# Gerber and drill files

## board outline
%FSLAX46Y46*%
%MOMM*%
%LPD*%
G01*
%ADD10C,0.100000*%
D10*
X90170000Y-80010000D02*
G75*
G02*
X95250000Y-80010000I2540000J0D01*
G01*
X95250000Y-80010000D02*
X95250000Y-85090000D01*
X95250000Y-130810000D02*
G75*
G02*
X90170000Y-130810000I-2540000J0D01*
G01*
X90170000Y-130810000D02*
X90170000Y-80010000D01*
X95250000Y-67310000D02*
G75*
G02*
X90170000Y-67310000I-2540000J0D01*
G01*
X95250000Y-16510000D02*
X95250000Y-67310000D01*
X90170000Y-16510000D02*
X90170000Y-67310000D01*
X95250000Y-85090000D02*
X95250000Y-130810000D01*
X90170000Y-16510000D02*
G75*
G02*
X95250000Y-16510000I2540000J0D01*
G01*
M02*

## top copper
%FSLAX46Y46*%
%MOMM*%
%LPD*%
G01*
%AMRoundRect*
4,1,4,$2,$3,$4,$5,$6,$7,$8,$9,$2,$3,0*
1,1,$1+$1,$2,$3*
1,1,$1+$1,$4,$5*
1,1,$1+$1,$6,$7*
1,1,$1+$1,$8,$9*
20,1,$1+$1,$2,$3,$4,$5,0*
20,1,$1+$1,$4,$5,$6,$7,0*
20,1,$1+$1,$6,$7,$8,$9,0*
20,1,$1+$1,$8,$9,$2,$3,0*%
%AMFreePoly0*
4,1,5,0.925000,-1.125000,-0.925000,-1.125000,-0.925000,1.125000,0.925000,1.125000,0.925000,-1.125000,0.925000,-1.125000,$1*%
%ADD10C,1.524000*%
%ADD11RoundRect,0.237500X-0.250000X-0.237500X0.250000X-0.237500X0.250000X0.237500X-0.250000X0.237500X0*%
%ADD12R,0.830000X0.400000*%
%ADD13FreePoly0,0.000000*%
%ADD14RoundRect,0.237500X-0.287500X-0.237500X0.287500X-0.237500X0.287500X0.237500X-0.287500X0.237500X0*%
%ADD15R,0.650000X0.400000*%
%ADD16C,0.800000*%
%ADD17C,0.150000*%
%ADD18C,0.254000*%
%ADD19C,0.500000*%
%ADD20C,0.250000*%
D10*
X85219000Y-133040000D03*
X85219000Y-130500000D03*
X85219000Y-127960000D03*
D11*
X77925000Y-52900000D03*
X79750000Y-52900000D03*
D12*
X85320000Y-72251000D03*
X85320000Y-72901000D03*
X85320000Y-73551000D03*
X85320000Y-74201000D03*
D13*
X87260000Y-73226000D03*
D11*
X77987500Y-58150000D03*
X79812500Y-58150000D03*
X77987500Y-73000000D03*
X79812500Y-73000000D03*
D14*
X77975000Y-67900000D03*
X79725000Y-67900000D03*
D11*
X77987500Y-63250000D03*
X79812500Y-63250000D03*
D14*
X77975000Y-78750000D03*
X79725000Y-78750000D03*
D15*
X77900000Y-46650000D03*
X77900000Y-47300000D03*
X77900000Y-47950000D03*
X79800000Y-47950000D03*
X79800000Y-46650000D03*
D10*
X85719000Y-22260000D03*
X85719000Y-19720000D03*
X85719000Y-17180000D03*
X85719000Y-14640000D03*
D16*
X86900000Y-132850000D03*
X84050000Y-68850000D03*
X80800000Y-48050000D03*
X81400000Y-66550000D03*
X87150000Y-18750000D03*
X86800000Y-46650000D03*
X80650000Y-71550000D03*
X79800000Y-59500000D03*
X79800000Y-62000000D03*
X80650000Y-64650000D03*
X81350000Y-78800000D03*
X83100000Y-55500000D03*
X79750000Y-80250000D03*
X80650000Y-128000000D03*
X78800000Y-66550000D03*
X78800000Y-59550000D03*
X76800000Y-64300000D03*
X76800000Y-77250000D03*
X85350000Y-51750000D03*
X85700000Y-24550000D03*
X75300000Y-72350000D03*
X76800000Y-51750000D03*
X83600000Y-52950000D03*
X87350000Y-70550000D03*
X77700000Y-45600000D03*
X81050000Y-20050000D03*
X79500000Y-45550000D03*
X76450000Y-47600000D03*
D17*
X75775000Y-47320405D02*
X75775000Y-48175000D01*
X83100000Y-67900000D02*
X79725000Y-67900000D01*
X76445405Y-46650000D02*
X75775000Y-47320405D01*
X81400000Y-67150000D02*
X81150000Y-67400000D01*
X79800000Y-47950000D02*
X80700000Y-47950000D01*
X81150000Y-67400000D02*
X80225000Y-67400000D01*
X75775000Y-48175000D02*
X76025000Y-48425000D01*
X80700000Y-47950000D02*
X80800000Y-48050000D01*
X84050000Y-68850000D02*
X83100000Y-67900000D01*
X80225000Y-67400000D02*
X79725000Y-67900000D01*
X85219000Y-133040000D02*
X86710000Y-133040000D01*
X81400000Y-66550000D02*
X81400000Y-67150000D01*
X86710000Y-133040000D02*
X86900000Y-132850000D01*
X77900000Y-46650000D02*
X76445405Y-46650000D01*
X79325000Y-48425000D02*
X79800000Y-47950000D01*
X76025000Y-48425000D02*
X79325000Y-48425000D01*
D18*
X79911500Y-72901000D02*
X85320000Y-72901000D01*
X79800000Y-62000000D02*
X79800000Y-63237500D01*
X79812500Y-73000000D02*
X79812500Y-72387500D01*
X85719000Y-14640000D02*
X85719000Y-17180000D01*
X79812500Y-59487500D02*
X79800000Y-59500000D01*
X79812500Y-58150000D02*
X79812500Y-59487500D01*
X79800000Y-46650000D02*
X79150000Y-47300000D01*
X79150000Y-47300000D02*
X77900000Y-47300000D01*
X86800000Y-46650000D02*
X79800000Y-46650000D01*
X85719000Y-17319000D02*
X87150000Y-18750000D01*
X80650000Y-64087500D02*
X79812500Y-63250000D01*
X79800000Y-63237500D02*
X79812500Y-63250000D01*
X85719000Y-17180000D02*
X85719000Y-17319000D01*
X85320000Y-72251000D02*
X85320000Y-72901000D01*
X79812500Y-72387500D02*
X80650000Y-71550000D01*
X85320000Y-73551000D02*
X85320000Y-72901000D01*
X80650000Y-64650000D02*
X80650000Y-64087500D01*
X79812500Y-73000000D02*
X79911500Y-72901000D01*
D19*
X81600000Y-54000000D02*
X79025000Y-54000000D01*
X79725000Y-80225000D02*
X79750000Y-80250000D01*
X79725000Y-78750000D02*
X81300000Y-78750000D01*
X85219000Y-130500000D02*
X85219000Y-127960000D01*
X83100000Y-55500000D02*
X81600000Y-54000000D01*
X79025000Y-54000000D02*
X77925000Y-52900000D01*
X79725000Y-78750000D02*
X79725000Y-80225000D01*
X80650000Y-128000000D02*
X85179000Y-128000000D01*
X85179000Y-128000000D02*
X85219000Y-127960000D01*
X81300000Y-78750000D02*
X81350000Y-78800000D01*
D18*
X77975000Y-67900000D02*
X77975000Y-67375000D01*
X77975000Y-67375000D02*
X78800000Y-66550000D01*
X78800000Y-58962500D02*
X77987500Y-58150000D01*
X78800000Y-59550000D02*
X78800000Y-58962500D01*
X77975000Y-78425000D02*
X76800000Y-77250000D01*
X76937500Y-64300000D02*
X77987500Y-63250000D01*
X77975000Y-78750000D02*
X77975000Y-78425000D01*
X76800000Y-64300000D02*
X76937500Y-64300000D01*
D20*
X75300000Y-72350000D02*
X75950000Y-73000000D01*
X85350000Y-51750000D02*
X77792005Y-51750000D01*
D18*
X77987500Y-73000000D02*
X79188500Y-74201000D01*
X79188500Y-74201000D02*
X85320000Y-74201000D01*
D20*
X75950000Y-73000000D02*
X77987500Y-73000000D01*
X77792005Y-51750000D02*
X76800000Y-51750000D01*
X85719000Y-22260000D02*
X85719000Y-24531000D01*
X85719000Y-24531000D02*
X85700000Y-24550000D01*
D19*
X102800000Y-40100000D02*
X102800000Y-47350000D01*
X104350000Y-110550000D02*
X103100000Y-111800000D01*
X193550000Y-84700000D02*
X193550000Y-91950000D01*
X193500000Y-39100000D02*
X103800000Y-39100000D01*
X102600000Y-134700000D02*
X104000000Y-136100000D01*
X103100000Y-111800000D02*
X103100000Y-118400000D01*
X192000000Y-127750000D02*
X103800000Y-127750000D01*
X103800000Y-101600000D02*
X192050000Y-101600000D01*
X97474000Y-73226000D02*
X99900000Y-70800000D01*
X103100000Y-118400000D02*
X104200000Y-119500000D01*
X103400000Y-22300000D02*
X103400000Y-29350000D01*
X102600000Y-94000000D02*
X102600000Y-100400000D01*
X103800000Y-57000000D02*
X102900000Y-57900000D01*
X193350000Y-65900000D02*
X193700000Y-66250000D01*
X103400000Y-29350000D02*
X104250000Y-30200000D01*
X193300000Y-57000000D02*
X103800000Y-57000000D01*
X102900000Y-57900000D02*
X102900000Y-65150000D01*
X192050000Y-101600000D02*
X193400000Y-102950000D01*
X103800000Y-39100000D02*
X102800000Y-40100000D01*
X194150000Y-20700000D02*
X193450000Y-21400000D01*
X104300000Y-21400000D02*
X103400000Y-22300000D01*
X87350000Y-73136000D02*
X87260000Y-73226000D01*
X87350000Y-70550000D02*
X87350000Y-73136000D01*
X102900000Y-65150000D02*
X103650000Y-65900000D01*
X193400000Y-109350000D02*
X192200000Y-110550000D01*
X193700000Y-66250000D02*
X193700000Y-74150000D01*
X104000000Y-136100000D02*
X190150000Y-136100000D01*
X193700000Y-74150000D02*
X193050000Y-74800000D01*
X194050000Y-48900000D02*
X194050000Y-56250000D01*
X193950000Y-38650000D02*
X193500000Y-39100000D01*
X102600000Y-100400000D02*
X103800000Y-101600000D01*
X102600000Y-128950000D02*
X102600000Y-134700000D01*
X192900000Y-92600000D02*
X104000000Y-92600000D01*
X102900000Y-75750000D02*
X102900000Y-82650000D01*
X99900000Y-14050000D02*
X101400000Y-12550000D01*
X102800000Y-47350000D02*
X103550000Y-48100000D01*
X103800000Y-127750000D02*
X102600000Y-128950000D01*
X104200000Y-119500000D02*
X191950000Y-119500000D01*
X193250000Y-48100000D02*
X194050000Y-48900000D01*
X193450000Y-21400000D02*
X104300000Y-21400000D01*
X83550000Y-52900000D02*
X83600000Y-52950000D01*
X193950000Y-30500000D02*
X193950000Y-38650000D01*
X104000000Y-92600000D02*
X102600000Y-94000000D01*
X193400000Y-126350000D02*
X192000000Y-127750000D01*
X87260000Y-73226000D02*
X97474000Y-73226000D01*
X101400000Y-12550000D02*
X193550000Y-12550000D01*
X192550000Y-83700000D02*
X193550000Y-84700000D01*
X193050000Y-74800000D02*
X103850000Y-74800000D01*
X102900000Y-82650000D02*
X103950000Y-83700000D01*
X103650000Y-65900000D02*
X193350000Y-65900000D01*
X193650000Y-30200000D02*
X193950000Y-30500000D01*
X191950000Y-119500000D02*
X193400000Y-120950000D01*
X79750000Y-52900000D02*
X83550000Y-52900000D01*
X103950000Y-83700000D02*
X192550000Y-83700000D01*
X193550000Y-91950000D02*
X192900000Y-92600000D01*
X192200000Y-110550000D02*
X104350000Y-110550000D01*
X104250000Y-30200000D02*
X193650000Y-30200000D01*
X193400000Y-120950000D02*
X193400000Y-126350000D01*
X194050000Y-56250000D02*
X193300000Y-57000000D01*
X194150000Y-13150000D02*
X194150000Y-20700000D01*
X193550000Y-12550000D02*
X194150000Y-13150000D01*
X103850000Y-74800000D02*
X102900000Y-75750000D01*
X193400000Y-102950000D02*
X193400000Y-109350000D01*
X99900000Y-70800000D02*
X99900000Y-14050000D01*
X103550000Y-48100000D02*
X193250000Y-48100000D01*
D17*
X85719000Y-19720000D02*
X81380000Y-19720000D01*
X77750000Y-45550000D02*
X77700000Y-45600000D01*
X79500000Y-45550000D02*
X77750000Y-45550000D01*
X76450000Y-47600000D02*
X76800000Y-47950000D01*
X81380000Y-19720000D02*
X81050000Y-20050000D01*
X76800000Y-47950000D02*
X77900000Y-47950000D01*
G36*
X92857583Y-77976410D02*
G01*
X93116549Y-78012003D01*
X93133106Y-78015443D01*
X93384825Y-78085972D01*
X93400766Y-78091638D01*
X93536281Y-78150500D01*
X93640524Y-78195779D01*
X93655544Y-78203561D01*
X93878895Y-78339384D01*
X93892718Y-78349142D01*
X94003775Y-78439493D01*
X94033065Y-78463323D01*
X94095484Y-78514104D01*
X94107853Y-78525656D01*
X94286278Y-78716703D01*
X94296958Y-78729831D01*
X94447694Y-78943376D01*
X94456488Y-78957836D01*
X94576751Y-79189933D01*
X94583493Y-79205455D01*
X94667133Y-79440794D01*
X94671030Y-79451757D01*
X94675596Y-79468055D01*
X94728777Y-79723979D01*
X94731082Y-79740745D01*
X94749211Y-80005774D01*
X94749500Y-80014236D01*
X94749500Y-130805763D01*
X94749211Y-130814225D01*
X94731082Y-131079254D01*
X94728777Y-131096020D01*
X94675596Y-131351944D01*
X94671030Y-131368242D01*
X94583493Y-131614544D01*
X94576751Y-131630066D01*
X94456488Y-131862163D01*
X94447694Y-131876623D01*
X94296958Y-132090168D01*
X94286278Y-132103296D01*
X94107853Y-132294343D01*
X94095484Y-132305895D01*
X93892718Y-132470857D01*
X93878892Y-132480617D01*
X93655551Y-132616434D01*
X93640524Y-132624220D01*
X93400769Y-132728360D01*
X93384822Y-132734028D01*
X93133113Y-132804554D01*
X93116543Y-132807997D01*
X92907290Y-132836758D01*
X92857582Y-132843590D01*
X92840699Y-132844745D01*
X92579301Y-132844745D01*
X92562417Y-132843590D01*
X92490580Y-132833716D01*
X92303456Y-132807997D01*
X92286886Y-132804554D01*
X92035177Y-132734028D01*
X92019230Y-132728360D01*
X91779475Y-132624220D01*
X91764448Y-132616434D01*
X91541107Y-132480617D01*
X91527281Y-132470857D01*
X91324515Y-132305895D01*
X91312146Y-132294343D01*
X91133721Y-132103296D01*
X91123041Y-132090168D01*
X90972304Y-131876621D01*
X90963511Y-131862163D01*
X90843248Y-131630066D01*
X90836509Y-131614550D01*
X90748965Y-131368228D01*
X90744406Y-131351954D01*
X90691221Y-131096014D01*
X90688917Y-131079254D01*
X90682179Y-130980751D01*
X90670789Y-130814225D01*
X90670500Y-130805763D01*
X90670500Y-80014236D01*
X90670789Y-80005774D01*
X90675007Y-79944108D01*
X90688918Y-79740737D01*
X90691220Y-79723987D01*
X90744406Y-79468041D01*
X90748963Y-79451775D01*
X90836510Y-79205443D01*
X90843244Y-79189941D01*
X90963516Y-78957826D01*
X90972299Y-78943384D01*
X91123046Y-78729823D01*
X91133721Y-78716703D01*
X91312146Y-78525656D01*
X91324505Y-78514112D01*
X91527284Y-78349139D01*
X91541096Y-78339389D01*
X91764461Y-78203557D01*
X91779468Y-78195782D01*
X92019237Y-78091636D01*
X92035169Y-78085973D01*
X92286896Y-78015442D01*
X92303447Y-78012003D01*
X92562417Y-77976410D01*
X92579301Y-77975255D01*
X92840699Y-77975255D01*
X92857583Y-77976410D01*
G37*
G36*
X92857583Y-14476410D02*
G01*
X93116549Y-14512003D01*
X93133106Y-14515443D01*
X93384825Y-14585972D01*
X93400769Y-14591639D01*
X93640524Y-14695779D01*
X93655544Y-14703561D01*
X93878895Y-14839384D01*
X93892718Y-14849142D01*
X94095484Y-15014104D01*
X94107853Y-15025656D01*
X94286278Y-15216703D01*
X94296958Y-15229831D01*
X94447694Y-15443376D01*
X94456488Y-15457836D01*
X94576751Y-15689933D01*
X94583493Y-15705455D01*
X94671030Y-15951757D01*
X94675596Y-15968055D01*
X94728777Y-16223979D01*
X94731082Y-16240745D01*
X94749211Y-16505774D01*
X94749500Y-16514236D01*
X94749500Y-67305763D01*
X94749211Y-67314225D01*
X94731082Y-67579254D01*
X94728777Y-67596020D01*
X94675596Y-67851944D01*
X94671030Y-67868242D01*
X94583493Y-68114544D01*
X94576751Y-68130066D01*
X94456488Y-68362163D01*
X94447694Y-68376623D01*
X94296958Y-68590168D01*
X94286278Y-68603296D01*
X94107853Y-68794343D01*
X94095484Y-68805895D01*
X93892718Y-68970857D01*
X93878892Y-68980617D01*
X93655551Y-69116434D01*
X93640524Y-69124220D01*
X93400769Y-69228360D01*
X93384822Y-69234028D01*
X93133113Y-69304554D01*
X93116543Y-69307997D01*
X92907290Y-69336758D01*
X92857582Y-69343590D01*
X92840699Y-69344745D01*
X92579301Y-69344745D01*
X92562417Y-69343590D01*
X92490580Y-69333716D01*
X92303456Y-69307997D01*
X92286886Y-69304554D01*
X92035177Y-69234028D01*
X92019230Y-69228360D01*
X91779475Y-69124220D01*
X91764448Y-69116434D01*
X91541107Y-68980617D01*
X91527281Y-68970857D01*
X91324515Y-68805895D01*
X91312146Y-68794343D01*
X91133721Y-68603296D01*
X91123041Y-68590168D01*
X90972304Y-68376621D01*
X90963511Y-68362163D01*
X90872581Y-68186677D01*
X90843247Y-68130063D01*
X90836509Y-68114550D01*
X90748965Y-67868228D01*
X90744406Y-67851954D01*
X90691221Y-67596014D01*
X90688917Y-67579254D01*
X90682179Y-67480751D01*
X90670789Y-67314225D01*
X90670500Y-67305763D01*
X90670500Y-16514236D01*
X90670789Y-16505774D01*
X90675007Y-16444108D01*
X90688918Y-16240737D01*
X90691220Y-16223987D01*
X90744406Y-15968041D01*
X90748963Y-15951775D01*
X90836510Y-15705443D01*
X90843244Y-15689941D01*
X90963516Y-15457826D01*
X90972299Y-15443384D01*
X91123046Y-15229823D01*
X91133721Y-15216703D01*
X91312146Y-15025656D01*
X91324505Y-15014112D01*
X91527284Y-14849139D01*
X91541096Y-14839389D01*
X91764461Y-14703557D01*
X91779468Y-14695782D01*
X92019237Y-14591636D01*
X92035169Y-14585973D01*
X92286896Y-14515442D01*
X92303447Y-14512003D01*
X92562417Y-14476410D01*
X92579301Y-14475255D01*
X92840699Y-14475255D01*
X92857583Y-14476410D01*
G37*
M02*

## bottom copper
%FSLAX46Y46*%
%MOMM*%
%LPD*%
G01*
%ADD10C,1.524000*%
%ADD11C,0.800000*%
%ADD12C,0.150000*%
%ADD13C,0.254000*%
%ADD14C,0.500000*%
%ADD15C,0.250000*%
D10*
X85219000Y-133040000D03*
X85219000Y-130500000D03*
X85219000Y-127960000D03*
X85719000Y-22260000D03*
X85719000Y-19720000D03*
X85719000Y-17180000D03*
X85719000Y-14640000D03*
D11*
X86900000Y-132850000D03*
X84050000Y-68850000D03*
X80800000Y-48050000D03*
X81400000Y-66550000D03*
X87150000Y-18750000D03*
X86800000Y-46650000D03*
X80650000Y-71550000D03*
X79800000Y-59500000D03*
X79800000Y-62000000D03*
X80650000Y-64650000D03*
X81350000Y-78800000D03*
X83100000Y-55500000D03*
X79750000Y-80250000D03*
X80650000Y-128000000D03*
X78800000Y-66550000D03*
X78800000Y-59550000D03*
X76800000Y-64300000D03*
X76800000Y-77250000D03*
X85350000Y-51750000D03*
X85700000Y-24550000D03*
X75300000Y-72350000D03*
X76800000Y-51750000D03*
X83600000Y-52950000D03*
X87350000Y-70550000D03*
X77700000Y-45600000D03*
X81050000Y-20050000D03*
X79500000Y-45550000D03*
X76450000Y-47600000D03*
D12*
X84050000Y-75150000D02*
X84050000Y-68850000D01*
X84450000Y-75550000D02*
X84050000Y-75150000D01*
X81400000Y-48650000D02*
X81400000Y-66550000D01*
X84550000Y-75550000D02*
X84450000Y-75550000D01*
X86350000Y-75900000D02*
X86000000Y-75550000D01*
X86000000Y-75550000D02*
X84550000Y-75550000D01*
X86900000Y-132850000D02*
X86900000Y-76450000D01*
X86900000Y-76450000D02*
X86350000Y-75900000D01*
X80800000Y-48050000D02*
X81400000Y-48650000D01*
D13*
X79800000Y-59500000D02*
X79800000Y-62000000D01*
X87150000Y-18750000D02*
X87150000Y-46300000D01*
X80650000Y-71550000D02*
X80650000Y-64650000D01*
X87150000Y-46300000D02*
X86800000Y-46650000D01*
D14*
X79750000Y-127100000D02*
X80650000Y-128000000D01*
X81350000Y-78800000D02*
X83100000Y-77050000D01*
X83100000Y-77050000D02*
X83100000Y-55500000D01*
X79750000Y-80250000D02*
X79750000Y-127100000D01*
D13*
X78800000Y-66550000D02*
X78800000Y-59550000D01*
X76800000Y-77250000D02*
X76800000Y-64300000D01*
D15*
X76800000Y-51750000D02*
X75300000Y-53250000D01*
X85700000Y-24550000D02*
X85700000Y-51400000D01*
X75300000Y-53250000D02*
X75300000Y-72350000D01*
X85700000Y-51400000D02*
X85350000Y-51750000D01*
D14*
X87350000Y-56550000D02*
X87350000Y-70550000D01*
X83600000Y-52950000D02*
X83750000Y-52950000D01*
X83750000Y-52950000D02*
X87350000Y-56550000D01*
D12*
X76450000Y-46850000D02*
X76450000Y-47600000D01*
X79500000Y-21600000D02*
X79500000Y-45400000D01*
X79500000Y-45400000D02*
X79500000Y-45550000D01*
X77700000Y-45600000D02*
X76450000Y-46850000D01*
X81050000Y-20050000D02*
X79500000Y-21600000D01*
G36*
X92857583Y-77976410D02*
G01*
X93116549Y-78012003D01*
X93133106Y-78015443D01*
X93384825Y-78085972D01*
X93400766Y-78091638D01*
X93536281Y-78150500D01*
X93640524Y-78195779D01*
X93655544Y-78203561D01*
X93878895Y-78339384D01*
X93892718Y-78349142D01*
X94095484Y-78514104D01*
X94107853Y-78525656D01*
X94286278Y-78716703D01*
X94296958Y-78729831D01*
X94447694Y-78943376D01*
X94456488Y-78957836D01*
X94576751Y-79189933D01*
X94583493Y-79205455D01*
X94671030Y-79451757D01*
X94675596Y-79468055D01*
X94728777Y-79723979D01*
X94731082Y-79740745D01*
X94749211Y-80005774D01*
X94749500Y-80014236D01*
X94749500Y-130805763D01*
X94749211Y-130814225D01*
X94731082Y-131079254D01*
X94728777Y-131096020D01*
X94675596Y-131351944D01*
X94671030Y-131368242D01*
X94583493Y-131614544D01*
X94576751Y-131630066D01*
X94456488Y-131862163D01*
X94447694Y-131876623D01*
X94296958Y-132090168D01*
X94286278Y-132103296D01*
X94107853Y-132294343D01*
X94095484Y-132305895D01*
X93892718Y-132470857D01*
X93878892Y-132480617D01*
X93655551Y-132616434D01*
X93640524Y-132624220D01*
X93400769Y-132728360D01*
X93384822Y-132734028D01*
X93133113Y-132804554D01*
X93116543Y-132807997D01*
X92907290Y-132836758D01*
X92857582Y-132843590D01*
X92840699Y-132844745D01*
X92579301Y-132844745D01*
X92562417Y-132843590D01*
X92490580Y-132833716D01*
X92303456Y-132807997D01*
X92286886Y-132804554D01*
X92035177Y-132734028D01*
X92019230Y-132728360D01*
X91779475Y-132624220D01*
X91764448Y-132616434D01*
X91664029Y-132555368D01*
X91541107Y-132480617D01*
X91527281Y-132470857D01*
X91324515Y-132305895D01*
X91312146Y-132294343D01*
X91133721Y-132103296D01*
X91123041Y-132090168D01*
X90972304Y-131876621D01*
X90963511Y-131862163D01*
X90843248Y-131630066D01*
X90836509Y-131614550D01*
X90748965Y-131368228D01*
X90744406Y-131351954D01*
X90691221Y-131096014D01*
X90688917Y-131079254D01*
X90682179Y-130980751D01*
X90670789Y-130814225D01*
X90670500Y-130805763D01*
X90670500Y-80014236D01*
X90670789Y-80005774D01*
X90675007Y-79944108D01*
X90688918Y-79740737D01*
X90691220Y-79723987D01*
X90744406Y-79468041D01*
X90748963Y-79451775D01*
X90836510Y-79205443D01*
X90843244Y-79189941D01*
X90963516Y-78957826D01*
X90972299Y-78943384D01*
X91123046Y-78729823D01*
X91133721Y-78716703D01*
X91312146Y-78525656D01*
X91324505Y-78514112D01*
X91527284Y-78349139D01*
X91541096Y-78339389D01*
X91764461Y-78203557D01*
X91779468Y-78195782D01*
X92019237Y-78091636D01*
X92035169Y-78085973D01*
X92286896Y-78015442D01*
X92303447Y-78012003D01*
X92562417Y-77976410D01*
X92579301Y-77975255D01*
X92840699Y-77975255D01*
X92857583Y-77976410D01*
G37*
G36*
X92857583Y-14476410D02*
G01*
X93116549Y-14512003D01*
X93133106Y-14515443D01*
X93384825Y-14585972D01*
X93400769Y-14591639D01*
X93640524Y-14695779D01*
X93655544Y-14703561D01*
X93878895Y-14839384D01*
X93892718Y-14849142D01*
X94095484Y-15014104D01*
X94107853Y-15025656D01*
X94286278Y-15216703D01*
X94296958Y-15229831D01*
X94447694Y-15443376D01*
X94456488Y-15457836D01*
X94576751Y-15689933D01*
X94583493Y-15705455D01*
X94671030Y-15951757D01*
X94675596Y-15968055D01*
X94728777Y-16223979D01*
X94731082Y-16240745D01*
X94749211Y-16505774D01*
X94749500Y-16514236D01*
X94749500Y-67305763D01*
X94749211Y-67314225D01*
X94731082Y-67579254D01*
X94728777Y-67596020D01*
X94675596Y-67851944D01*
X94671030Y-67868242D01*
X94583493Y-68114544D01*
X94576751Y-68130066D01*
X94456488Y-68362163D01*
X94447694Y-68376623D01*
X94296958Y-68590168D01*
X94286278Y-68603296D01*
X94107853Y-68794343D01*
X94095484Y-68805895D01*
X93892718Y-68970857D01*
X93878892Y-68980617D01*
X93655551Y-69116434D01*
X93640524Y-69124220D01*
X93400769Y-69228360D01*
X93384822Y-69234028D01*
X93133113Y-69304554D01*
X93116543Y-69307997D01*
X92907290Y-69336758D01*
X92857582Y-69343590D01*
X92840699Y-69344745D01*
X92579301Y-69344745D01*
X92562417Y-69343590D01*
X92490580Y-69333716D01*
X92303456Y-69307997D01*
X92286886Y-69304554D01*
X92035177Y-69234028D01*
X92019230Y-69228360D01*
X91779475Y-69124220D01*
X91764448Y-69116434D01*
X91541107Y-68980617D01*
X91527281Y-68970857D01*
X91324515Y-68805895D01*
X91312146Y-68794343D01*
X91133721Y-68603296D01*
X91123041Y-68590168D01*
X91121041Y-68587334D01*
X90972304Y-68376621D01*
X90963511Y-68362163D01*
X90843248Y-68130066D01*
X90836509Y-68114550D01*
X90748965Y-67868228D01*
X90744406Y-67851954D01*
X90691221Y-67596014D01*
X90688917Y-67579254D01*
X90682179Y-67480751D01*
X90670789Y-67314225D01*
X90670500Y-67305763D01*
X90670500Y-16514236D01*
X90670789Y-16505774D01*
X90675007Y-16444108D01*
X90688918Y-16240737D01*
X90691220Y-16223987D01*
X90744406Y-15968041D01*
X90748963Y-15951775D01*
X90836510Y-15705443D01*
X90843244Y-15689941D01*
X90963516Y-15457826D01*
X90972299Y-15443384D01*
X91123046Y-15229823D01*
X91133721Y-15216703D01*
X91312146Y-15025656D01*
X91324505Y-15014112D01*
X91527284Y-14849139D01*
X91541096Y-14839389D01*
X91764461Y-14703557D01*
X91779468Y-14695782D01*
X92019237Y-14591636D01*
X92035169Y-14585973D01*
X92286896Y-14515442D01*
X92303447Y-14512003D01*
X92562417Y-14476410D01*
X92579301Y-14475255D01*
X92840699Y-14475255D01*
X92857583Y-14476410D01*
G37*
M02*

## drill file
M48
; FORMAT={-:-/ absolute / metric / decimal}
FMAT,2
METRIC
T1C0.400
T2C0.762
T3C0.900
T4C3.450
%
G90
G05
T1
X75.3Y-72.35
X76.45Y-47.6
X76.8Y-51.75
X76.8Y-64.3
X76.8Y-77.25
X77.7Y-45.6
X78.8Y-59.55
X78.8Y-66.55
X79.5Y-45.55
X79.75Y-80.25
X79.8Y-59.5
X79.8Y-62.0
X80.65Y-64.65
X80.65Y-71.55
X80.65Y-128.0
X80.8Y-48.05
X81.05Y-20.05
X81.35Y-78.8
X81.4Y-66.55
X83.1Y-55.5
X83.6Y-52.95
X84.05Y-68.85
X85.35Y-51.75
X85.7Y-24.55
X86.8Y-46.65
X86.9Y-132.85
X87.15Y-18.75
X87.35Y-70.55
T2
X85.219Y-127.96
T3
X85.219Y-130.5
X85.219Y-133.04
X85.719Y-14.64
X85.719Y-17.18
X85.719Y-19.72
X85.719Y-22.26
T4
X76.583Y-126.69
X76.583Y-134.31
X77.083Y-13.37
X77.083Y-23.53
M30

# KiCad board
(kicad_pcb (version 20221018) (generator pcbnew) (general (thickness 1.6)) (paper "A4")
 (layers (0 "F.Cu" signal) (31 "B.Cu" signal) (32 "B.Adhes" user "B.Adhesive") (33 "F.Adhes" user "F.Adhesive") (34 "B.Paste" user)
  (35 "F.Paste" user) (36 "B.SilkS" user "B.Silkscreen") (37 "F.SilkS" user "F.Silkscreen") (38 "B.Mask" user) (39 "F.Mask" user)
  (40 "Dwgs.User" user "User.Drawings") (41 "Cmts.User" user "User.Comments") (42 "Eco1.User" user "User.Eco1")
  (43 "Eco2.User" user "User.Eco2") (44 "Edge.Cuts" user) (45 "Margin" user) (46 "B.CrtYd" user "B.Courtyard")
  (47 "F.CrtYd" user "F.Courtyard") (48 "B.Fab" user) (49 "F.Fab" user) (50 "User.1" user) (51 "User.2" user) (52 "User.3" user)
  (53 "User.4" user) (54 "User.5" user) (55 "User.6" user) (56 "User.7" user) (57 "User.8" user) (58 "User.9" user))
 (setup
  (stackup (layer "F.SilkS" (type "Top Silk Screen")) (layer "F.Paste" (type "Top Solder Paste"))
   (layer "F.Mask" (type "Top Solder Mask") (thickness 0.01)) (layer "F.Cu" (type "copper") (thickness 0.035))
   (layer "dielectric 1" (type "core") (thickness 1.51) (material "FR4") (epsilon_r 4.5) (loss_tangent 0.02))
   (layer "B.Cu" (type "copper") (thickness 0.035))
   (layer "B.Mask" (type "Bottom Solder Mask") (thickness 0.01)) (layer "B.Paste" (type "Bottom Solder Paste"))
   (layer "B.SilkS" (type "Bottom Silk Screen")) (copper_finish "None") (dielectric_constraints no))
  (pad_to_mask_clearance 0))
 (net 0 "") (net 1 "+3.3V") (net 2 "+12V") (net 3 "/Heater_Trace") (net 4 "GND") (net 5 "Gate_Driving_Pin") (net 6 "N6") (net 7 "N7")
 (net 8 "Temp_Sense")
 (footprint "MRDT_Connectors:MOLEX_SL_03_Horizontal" (layer "F.Cu") (at 85.219 133.04 90)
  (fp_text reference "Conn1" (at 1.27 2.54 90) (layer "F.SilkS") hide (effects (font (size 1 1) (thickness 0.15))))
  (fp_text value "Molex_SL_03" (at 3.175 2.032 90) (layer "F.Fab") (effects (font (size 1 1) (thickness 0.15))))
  (pad "" np_thru_hole circle (at -1.27 -8.636 90) (size 3.45 3.45) (drill 3.45) (layers "*.Cu" "*.Mask"))
  (pad "" np_thru_hole circle (at 6.35 -8.636 90) (size 3.45 3.45) (drill 3.45) (layers "*.Cu" "*.Mask"))
  (pad "1" thru_hole circle (at 0 0 90) (size 1.524 1.524) (drill 0.9) (layers "*.Cu" "*.Mask") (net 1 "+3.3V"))
  (pad "2" thru_hole circle (at 2.54 0 90) (size 1.524 1.524) (drill 0.9) (layers "*.Cu" "*.Mask") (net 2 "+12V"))
  (pad "3" thru_hole circle (at 5.08 0 90) (size 1.524 1.524) (drill 0.762) (layers "*.Cu" "*.Mask") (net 2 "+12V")))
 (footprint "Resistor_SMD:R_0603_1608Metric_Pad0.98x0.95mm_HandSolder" (layer "F.Cu") (at 78.8375 52.9)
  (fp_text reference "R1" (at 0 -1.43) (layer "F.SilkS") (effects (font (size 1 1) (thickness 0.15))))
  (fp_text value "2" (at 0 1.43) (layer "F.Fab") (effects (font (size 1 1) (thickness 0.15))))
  (pad "1" smd roundrect (at -0.9125 0) (size 0.975 0.95) (layers "F.Cu" "F.Paste" "F.Mask") (roundrect_rratio 0.25) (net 2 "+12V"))
  (pad "2" smd roundrect (at 0.9125 0) (size 0.975 0.95) (layers "F.Cu" "F.Paste" "F.Mask") (roundrect_rratio 0.25) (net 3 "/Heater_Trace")))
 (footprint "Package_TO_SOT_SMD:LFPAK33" (layer "F.Cu") (at 86.855 73.226) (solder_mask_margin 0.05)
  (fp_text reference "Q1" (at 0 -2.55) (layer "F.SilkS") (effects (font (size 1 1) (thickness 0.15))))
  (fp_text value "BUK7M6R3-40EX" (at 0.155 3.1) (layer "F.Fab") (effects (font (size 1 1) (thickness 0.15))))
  (pad "" smd rect (at -1.535 -0.975) (size 0.83 0.3) (layers "F.Paste"))
  (pad "" smd rect (at -1.535 -0.325) (size 0.83 0.3) (layers "F.Paste"))
  (pad "" smd rect (at -1.535 0.325) (size 0.83 0.3) (layers "F.Paste"))
  (pad "" smd rect (at -1.535 0.975) (size 0.83 0.3) (layers "F.Paste"))
  (pad "" smd rect (at -0.215 -0.626) (size 0.51 0.635) (layers "F.Paste"))
  (pad "" smd rect (at -0.215 0.626) (size 0.51 0.635) (layers "F.Paste"))
  (pad "" smd rect (at 0.645 -0.626) (size 0.51 0.635) (layers "F.Paste"))
  (pad "" smd rect (at 0.645 0.626) (size 0.51 0.635) (layers "F.Paste"))
  (pad "" smd rect (at 1.575 -0.975) (size 0.75 0.3) (layers "F.Paste"))
  (pad "" smd rect (at 1.575 -0.325) (size 0.75 0.3) (layers "F.Paste"))
  (pad "" smd rect (at 1.575 0.325) (size 0.75 0.3) (layers "F.Paste"))
  (pad "" smd rect (at 1.575 0.975) (size 0.75 0.3) (layers "F.Paste"))
  (pad "1" smd rect (at -1.535 -0.975) (size 0.83 0.4) (layers "F.Cu" "F.Mask") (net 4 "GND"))
  (pad "2" smd rect (at -1.535 -0.325) (size 0.83 0.4) (layers "F.Cu" "F.Mask") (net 4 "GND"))
  (pad "3" smd rect (at -1.535 0.325) (size 0.83 0.4) (layers "F.Cu" "F.Mask") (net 4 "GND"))
  (pad "4" smd rect (at -1.535 0.975) (size 0.83 0.4) (layers "F.Cu" "F.Mask") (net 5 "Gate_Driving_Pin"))
  (pad "5" smd custom (at 0.405 0) (size 1.85 2.25) (layers "F.Cu" "F.Mask") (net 3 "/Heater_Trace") (zone_connect 2)
   (thermal_bridge_angle 45) (options (clearance outline) (anchor rect)) (primitives)))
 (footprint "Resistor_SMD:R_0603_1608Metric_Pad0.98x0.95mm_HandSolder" (layer "F.Cu") (at 78.9 58.15)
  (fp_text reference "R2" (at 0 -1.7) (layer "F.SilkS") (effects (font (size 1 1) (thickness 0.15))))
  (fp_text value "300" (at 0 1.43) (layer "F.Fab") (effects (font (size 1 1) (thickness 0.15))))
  (pad "1" smd roundrect (at -0.9125 0) (size 0.975 0.95) (layers "F.Cu" "F.Paste" "F.Mask") (roundrect_rratio 0.25) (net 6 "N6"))
  (pad "2" smd roundrect (at 0.9125 0) (size 0.975 0.95) (layers "F.Cu" "F.Paste" "F.Mask") (roundrect_rratio 0.25) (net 4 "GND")))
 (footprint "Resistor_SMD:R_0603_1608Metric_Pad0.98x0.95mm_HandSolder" (layer "F.Cu") (at 78.9 73)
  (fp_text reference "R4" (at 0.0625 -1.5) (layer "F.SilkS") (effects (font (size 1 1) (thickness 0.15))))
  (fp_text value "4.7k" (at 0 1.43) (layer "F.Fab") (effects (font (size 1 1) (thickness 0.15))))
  (pad "1" smd roundrect (at -0.9125 0) (size 0.975 0.95) (layers "F.Cu" "F.Paste" "F.Mask") (roundrect_rratio 0.25)
   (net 5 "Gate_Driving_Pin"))
  (pad "2" smd roundrect (at 0.9125 0) (size 0.975 0.95) (layers "F.Cu" "F.Paste" "F.Mask") (roundrect_rratio 0.25) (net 4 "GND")))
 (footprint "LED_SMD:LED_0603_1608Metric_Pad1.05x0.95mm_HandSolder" (layer "F.Cu") (at 78.85 67.9)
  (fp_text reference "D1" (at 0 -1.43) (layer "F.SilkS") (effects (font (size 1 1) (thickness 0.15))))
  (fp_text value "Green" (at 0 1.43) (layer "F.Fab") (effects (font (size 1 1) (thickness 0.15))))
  (pad "1" smd roundrect (at -0.875 0) (size 1.05 0.95) (layers "F.Cu" "F.Paste" "F.Mask") (roundrect_rratio 0.25) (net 6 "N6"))
  (pad "2" smd roundrect (at 0.875 0) (size 1.05 0.95) (layers "F.Cu" "F.Paste" "F.Mask") (roundrect_rratio 0.25) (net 1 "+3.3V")))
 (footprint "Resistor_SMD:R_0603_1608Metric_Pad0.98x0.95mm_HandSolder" (layer "F.Cu") (at 78.9 63.25)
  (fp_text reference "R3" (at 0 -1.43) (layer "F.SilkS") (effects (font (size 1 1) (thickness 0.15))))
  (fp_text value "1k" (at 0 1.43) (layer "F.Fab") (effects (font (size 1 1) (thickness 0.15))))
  (pad "1" smd roundrect (at -0.9125 0) (size 0.975 0.95) (layers "F.Cu" "F.Paste" "F.Mask") (roundrect_rratio 0.25) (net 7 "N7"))
  (pad "2" smd roundrect (at 0.9125 0) (size 0.975 0.95) (layers "F.Cu" "F.Paste" "F.Mask") (roundrect_rratio 0.25) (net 4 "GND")))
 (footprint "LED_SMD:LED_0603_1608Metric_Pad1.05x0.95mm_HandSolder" (layer "F.Cu") (at 78.85 78.75)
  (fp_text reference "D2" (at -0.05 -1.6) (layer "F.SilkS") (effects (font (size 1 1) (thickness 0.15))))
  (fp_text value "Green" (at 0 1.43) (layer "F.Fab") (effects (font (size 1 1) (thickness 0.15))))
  (pad "1" smd roundrect (at -0.875 0) (size 1.05 0.95) (layers "F.Cu" "F.Paste" "F.Mask") (roundrect_rratio 0.25) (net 7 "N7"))
  (pad "2" smd roundrect (at 0.875 0) (size 1.05 0.95) (layers "F.Cu" "F.Paste" "F.Mask") (roundrect_rratio 0.25) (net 2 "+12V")))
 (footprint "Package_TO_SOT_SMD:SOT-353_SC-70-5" (layer "F.Cu") (at 78.85 47.3)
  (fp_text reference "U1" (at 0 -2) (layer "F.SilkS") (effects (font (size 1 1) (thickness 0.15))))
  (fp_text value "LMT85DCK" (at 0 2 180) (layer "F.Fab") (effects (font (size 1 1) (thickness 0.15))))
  (pad "1" smd rect (at -0.95 -0.65) (size 0.65 0.4) (layers "F.Cu" "F.Paste" "F.Mask") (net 1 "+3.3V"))
  (pad "2" smd rect (at -0.95 0) (size 0.65 0.4) (layers "F.Cu" "F.Paste" "F.Mask") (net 4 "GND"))
  (pad "3" smd rect (at -0.95 0.65) (size 0.65 0.4) (layers "F.Cu" "F.Paste" "F.Mask") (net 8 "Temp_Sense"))
  (pad "4" smd rect (at 0.95 0.65) (size 0.65 0.4) (layers "F.Cu" "F.Paste" "F.Mask") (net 1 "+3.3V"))
  (pad "5" smd rect (at 0.95 -0.65) (size 0.65 0.4) (layers "F.Cu" "F.Paste" "F.Mask") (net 4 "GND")))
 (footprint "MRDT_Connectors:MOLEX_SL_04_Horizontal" (layer "F.Cu") (at 85.719 22.26 90)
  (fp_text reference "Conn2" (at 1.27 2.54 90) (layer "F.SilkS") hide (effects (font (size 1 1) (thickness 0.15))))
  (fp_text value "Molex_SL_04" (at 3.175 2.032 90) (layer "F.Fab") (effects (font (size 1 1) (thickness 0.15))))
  (pad "" np_thru_hole circle (at -1.27 -8.636 90) (size 3.45 3.45) (drill 3.45) (layers "*.Cu" "*.Mask"))
  (pad "" np_thru_hole circle (at 8.89 -8.636 90) (size 3.45 3.45) (drill 3.45) (layers "*.Cu" "*.Mask"))
  (pad "1" thru_hole circle (at 0 0 90) (size 1.524 1.524) (drill 0.9) (layers "*.Cu" "*.Mask") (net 5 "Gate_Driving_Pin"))
  (pad "2" thru_hole circle (at 2.54 0 90) (size 1.524 1.524) (drill 0.9) (layers "*.Cu" "*.Mask") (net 8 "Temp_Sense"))
  (pad "3" thru_hole circle (at 5.08 0 90) (size 1.524 1.524) (drill 0.9) (layers "*.Cu" "*.Mask") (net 4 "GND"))
  (pad "4" thru_hole circle (at 7.62 0 90) (size 1.524 1.524) (drill 0.9) (layers "*.Cu" "*.Mask") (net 4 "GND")))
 (gr_arc (start 90.17 80.01) (mid 92.71 77.47) (end 95.25 80.01) (stroke (width 0.1) (type default)) (layer "Edge.Cuts"))
 (gr_line (start 95.25 80.01) (end 95.25 85.09) (stroke (width 0.1) (type default)) (layer "Edge.Cuts"))
 (gr_arc (start 95.25 130.81) (mid 92.71 133.35) (end 90.17 130.81) (stroke (width 0.1) (type default)) (layer "Edge.Cuts"))
 (gr_line (start 90.17 130.81) (end 90.17 80.01) (stroke (width 0.1) (type default)) (layer "Edge.Cuts"))
 (gr_arc (start 95.25 67.31) (mid 92.71 69.85) (end 90.17 67.31) (stroke (width 0.1) (type default)) (layer "Edge.Cuts"))
 (gr_line (start 95.25 16.51) (end 95.25 67.31) (stroke (width 0.1) (type default)) (layer "Edge.Cuts"))
 (gr_line (start 90.17 16.51) (end 90.17 67.31) (stroke (width 0.1) (type default)) (layer "Edge.Cuts"))
 (gr_line (start 95.25 85.09) (end 95.25 130.81) (stroke (width 0.1) (type default)) (layer "Edge.Cuts"))
 (gr_arc (start 90.17 16.51) (mid 92.71 13.97) (end 95.25 16.51) (stroke (width 0.1) (type default)) (layer "Edge.Cuts"))
 (segment (start 75.775 47.320405) (end 75.775 48.175) (width 0.15) (layer "F.Cu") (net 1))
 (segment (start 83.1 67.9) (end 79.725 67.9) (width 0.15) (layer "F.Cu") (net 1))
 (segment (start 76.445405 46.65) (end 75.775 47.320405) (width 0.15) (layer "F.Cu") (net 1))
 (segment (start 81.4 67.15) (end 81.15 67.4) (width 0.15) (layer "F.Cu") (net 1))
 (segment (start 79.8 47.95) (end 80.7 47.95) (width 0.15) (layer "F.Cu") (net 1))
 (segment (start 81.15 67.4) (end 80.225 67.4) (width 0.15) (layer "F.Cu") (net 1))
 (segment (start 75.775 48.175) (end 76.025 48.425) (width 0.15) (layer "F.Cu") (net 1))
 (segment (start 80.7 47.95) (end 80.8 48.05) (width 0.15) (layer "F.Cu") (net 1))
 (segment (start 84.05 68.85) (end 83.1 67.9) (width 0.15) (layer "F.Cu") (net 1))
 (segment (start 80.225 67.4) (end 79.725 67.9) (width 0.15) (layer "F.Cu") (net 1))
 (segment (start 85.219 133.04) (end 86.71 133.04) (width 0.15) (layer "F.Cu") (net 1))
 (segment (start 81.4 66.55) (end 81.4 67.15) (width 0.15) (layer "F.Cu") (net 1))
 (segment (start 86.71 133.04) (end 86.9 132.85) (width 0.15) (layer "F.Cu") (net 1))
 (segment (start 77.9 46.65) (end 76.445405 46.65) (width 0.15) (layer "F.Cu") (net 1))
 (segment (start 79.325 48.425) (end 79.8 47.95) (width 0.15) (layer "F.Cu") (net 1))
 (segment (start 76.025 48.425) (end 79.325 48.425) (width 0.15) (layer "F.Cu") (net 1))
 (via (at 86.9 132.85) (size 0.8) (drill 0.4) (layers "F.Cu" "B.Cu") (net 1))
 (via (at 84.05 68.85) (size 0.8) (drill 0.4) (layers "F.Cu" "B.Cu") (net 1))
 (via (at 80.8 48.05) (size 0.8) (drill 0.4) (layers "F.Cu" "B.Cu") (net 1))
 (via (at 81.4 66.55) (size 0.8) (drill 0.4) (layers "F.Cu" "B.Cu") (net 1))
 (segment (start 84.05 75.15) (end 84.05 68.85) (width 0.15) (layer "B.Cu") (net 1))
 (segment (start 84.45 75.55) (end 84.05 75.15) (width 0.15) (layer "B.Cu") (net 1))
 (segment (start 81.4 48.65) (end 81.4 66.55) (width 0.15) (layer "B.Cu") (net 1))
 (segment (start 84.55 75.55) (end 84.45 75.55) (width 0.15) (layer "B.Cu") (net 1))
 (segment (start 86.35 75.9) (end 86 75.55) (width 0.15) (layer "B.Cu") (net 1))
 (segment (start 86 75.55) (end 84.55 75.55) (width 0.15) (layer "B.Cu") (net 1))
 (segment (start 86.9 132.85) (end 86.9 76.45) (width 0.15) (layer "B.Cu") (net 1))
 (segment (start 86.9 76.45) (end 86.35 75.9) (width 0.15) (layer "B.Cu") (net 1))
 (segment (start 80.8 48.05) (end 81.4 48.65) (width 0.15) (layer "B.Cu") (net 1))
 (segment (start 79.9115 72.901) (end 85.32 72.901) (width 0.254) (layer "F.Cu") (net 4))
 (segment (start 79.8 62) (end 79.8 63.2375) (width 0.254) (layer "F.Cu") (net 4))
 (segment (start 79.8125 73) (end 79.8125 72.3875) (width 0.254) (layer "F.Cu") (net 4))
 (segment (start 85.719 14.64) (end 85.719 17.18) (width 0.254) (layer "F.Cu") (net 4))
 (segment (start 79.8125 59.4875) (end 79.8 59.5) (width 0.254) (layer "F.Cu") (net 4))
 (segment (start 79.8125 58.15) (end 79.8125 59.4875) (width 0.254) (layer "F.Cu") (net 4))
 (segment (start 79.8 46.65) (end 79.15 47.3) (width 0.254) (layer "F.Cu") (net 4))
 (segment (start 79.15 47.3) (end 77.9 47.3) (width 0.254) (layer "F.Cu") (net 4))
 (segment (start 86.8 46.65) (end 79.8 46.65) (width 0.254) (layer "F.Cu") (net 4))
 (segment (start 85.719 17.319) (end 87.15 18.75) (width 0.254) (layer "F.Cu") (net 4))
 (segment (start 80.65 64.0875) (end 79.8125 63.25) (width 0.254) (layer "F.Cu") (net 4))
 (segment (start 79.8 63.2375) (end 79.8125 63.25) (width 0.254) (layer "F.Cu") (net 4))
 (segment (start 85.719 17.18) (end 85.719 17.319) (width 0.254) (layer "F.Cu") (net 4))
 (segment (start 85.32 72.251) (end 85.32 72.901) (width 0.254) (layer "F.Cu") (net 4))
 (segment (start 79.8125 72.3875) (end 80.65 71.55) (width 0.254) (layer "F.Cu") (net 4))
 (segment (start 85.32 73.551) (end 85.32 72.901) (width 0.254) (layer "F.Cu") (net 4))
 (segment (start 80.65 64.65) (end 80.65 64.0875) (width 0.254) (layer "F.Cu") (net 4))
 (segment (start 79.8125 73) (end 79.9115 72.901) (width 0.254) (layer "F.Cu") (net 4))
 (via (at 87.15 18.75) (size 0.8) (drill 0.4) (layers "F.Cu" "B.Cu") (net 4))
 (via (at 86.8 46.65) (size 0.8) (drill 0.4) (layers "F.Cu" "B.Cu") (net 4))
 (via (at 80.65 71.55) (size 0.8) (drill 0.4) (layers "F.Cu" "B.Cu") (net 4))
 (via (at 79.8 59.5) (size 0.8) (drill 0.4) (layers "F.Cu" "B.Cu") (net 4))
 (via (at 79.8 62) (size 0.8) (drill 0.4) (layers "F.Cu" "B.Cu") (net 4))
 (via (at 80.65 64.65) (size 0.8) (drill 0.4) (layers "F.Cu" "B.Cu") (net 4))
 (segment (start 79.8 59.5) (end 79.8 62) (width 0.254) (layer "B.Cu") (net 4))
 (segment (start 87.15 18.75) (end 87.15 46.3) (width 0.254) (layer "B.Cu") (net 4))
 (segment (start 80.65 71.55) (end 80.65 64.65) (width 0.254) (layer "B.Cu") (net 4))
 (segment (start 87.15 46.3) (end 86.8 46.65) (width 0.254) (layer "B.Cu") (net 4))
 (segment (start 81.6 54) (end 79.025 54) (width 0.5) (layer "F.Cu") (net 2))
 (segment (start 79.725 80.225) (end 79.75 80.25) (width 0.5) (layer "F.Cu") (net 2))
 (segment (start 79.725 78.75) (end 81.3 78.75) (width 0.5) (layer "F.Cu") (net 2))
 (segment (start 85.219 130.5) (end 85.219 127.96) (width 0.5) (layer "F.Cu") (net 2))
 (segment (start 83.1 55.5) (end 81.6 54) (width 0.5) (layer "F.Cu") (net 2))
 (segment (start 79.025 54) (end 77.925 52.9) (width 0.5) (layer "F.Cu") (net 2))
 (segment (start 79.725 78.75) (end 79.725 80.225) (width 0.5) (layer "F.Cu") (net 2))
 (segment (start 80.65 128) (end 85.179 128) (width 0.5) (layer "F.Cu") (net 2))
 (segment (start 85.179 128) (end 85.219 127.96) (width 0.5) (layer "F.Cu") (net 2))
 (segment (start 81.3 78.75) (end 81.35 78.8) (width 0.5) (layer "F.Cu") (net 2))
 (via (at 81.35 78.8) (size 0.8) (drill 0.4) (layers "F.Cu" "B.Cu") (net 2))
 (via (at 83.1 55.5) (size 0.8) (drill 0.4) (layers "F.Cu" "B.Cu") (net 2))
 (via (at 79.75 80.25) (size 0.8) (drill 0.4) (layers "F.Cu" "B.Cu") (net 2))
 (via (at 80.65 128) (size 0.8) (drill 0.4) (layers "F.Cu" "B.Cu") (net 2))
 (segment (start 79.75 127.1) (end 80.65 128) (width 0.5) (layer "B.Cu") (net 2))
 (segment (start 81.35 78.8) (end 83.1 77.05) (width 0.5) (layer "B.Cu") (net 2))
 (segment (start 83.1 77.05) (end 83.1 55.5) (width 0.5) (layer "B.Cu") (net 2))
 (segment (start 79.75 80.25) (end 79.75 127.1) (width 0.5) (layer "B.Cu") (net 2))
 (segment (start 77.975 67.9) (end 77.975 67.375) (width 0.254) (layer "F.Cu") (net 6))
 (segment (start 77.975 67.375) (end 78.8 66.55) (width 0.254) (layer "F.Cu") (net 6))
 (segment (start 78.8 58.9625) (end 77.9875 58.15) (width 0.254) (layer "F.Cu") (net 6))
 (segment (start 78.8 59.55) (end 78.8 58.9625) (width 0.254) (layer "F.Cu") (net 6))
 (via (at 78.8 66.55) (size 0.8) (drill 0.4) (layers "F.Cu" "B.Cu") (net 6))
 (via (at 78.8 59.55) (size 0.8) (drill 0.4) (layers "F.Cu" "B.Cu") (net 6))
 (segment (start 78.8 66.55) (end 78.8 59.55) (width 0.254) (layer "B.Cu") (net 6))
 (segment (start 77.975 78.425) (end 76.8 77.25) (width 0.254) (layer "F.Cu") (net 7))
 (segment (start 76.9375 64.3) (end 77.9875 63.25) (width 0.254) (layer "F.Cu") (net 7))
 (segment (start 77.975 78.75) (end 77.975 78.425) (width 0.254) (layer "F.Cu") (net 7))
 (segment (start 76.8 64.3) (end 76.9375 64.3) (width 0.254) (layer "F.Cu") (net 7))
 (via (at 76.8 64.3) (size 0.8) (drill 0.4) (layers "F.Cu" "B.Cu") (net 7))
 (via (at 76.8 77.25) (size 0.8) (drill 0.4) (layers "F.Cu" "B.Cu") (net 7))
 (segment (start 76.8 77.25) (end 76.8 64.3) (width 0.254) (layer "B.Cu") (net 7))
 (segment (start 75.3 72.35) (end 75.95 73) (width 0.25) (layer "F.Cu") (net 5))
 (segment (start 85.35 51.75) (end 77.792005 51.75) (width 0.25) (layer "F.Cu") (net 5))
 (segment (start 77.9875 73) (end 79.1885 74.201) (width 0.254) (layer "F.Cu") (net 5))
 (segment (start 79.1885 74.201) (end 85.32 74.201) (width 0.254) (layer "F.Cu") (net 5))
 (segment (start 75.95 73) (end 77.9875 73) (width 0.25) (layer "F.Cu") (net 5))
 (segment (start 77.792005 51.75) (end 76.8 51.75) (width 0.25) (layer "F.Cu") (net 5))
 (segment (start 85.719 22.26) (end 85.719 24.531) (width 0.25) (layer "F.Cu") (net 5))
 (segment (start 85.719 24.531) (end 85.7 24.55) (width 0.25) (layer "F.Cu") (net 5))
 (via (at 85.35 51.75) (size 0.8) (drill 0.4) (layers "F.Cu" "B.Cu") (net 5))
 (via (at 85.7 24.55) (size 0.8) (drill 0.4) (layers "F.Cu" "B.Cu") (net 5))
 (via (at 75.3 72.35) (size 0.8) (drill 0.4) (layers "F.Cu" "B.Cu") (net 5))
 (via (at 76.8 51.75) (size 0.8) (drill 0.4) (layers "F.Cu" "B.Cu") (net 5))
 (segment (start 76.8 51.75) (end 75.3 53.25) (width 0.25) (layer "B.Cu") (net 5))
 (segment (start 85.7 24.55) (end 85.7 51.4) (width 0.25) (layer "B.Cu") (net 5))
 (segment (start 75.3 53.25) (end 75.3 72.35) (width 0.25) (layer "B.Cu") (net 5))
 (segment (start 85.7 51.4) (end 85.35 51.75) (width 0.25) (layer "B.Cu") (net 5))
 (segment (start 102.8 40.1) (end 102.8 47.35) (width 0.5) (layer "F.Cu") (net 3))
 (segment (start 104.35 110.55) (end 103.1 111.8) (width 0.5) (layer "F.Cu") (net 3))
 (segment (start 193.55 84.7) (end 193.55 91.95) (width 0.5) (layer "F.Cu") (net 3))
 (segment (start 193.5 39.1) (end 103.8 39.1) (width 0.5) (layer "F.Cu") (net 3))
 (segment (start 102.6 134.7) (end 104 136.1) (width 0.5) (layer "F.Cu") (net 3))
 (segment (start 103.1 111.8) (end 103.1 118.4) (width 0.5) (layer "F.Cu") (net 3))
 (segment (start 192 127.75) (end 103.8 127.75) (width 0.5) (layer "F.Cu") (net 3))
 (segment (start 103.8 101.6) (end 192.05 101.6) (width 0.5) (layer "F.Cu") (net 3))
 (segment (start 97.474 73.226) (end 99.9 70.8) (width 0.5) (layer "F.Cu") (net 3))
 (segment (start 103.1 118.4) (end 104.2 119.5) (width 0.5) (layer "F.Cu") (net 3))
 (segment (start 103.4 22.3) (end 103.4 29.35) (width 0.5) (layer "F.Cu") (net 3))
 (segment (start 102.6 94) (end 102.6 100.4) (width 0.5) (layer "F.Cu") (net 3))
 (segment (start 103.8 57) (end 102.9 57.9) (width 0.5) (layer "F.Cu") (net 3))
 (segment (start 193.35 65.9) (end 193.7 66.25) (width 0.5) (layer "F.Cu") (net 3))
 (segment (start 103.4 29.35) (end 104.25 30.2) (width 0.5) (layer "F.Cu") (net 3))
 (segment (start 193.3 57) (end 103.8 57) (width 0.5) (layer "F.Cu") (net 3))
 (segment (start 102.9 57.9) (end 102.9 65.15) (width 0.5) (layer "F.Cu") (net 3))
 (segment (start 192.05 101.6) (end 193.4 102.95) (width 0.5) (layer "F.Cu") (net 3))
 (segment (start 103.8 39.1) (end 102.8 40.1) (width 0.5) (layer "F.Cu") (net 3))
 (segment (start 194.15 20.7) (end 193.45 21.4) (width 0.5) (layer "F.Cu") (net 3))
 (segment (start 104.3 21.4) (end 103.4 22.3) (width 0.5) (layer "F.Cu") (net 3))
 (segment (start 87.35 73.136) (end 87.26 73.226) (width 0.5) (layer "F.Cu") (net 3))
 (segment (start 87.35 70.55) (end 87.35 73.136) (width 0.5) (layer "F.Cu") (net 3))
 (segment (start 102.9 65.15) (end 103.65 65.9) (width 0.5) (layer "F.Cu") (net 3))
 (segment (start 193.4 109.35) (end 192.2 110.55) (width 0.5) (layer "F.Cu") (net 3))
 (segment (start 193.7 66.25) (end 193.7 74.15) (width 0.5) (layer "F.Cu") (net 3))
 (segment (start 104 136.1) (end 190.15 136.1) (width 0.5) (layer "F.Cu") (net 3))
 (segment (start 193.7 74.15) (end 193.05 74.8) (width 0.5) (layer "F.Cu") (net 3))
 (segment (start 194.05 48.9) (end 194.05 56.25) (width 0.5) (layer "F.Cu") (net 3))
 (segment (start 193.95 38.65) (end 193.5 39.1) (width 0.5) (layer "F.Cu") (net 3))
 (segment (start 102.6 100.4) (end 103.8 101.6) (width 0.5) (layer "F.Cu") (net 3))
 (segment (start 102.6 128.95) (end 102.6 134.7) (width 0.5) (layer "F.Cu") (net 3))
 (segment (start 192.9 92.6) (end 104 92.6) (width 0.5) (layer "F.Cu") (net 3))
 (segment (start 102.9 75.75) (end 102.9 82.65) (width 0.5) (layer "F.Cu") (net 3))
 (segment (start 99.9 14.05) (end 101.4 12.55) (width 0.5) (layer "F.Cu") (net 3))
 (segment (start 102.8 47.35) (end 103.55 48.1) (width 0.5) (layer "F.Cu") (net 3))
 (segment (start 103.8 127.75) (end 102.6 128.95) (width 0.5) (layer "F.Cu") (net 3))
 (segment (start 104.2 119.5) (end 191.95 119.5) (width 0.5) (layer "F.Cu") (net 3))
 (segment (start 193.25 48.1) (end 194.05 48.9) (width 0.5) (layer "F.Cu") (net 3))
 (segment (start 193.45 21.4) (end 104.3 21.4) (width 0.5) (layer "F.Cu") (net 3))
 (segment (start 83.55 52.9) (end 83.6 52.95) (width 0.5) (layer "F.Cu") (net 3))
 (segment (start 193.95 30.5) (end 193.95 38.65) (width 0.5) (layer "F.Cu") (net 3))
 (segment (start 104 92.6) (end 102.6 94) (width 0.5) (layer "F.Cu") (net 3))
 (segment (start 193.4 126.35) (end 192 127.75) (width 0.5) (layer "F.Cu") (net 3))
 (segment (start 87.26 73.226) (end 97.474 73.226) (width 0.5) (layer "F.Cu") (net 3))
 (segment (start 101.4 12.55) (end 193.55 12.55) (width 0.5) (layer "F.Cu") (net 3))
 (segment (start 192.55 83.7) (end 193.55 84.7) (width 0.5) (layer "F.Cu") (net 3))
 (segment (start 193.05 74.8) (end 103.85 74.8) (width 0.5) (layer "F.Cu") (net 3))
 (segment (start 102.9 82.65) (end 103.95 83.7) (width 0.5) (layer "F.Cu") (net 3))
 (segment (start 103.65 65.9) (end 193.35 65.9) (width 0.5) (layer "F.Cu") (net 3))
 (segment (start 193.65 30.2) (end 193.95 30.5) (width 0.5) (layer "F.Cu") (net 3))
 (segment (start 191.95 119.5) (end 193.4 120.95) (width 0.5) (layer "F.Cu") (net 3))
 (segment (start 79.75 52.9) (end 83.55 52.9) (width 0.5) (layer "F.Cu") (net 3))
 (segment (start 103.95 83.7) (end 192.55 83.7) (width 0.5) (layer "F.Cu") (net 3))
 (segment (start 193.55 91.95) (end 192.9 92.6) (width 0.5) (layer "F.Cu") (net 3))
 (segment (start 192.2 110.55) (end 104.35 110.55) (width 0.5) (layer "F.Cu") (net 3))
 (segment (start 104.25 30.2) (end 193.65 30.2) (width 0.5) (layer "F.Cu") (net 3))
 (segment (start 193.4 120.95) (end 193.4 126.35) (width 0.5) (layer "F.Cu") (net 3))
 (segment (start 194.05 56.25) (end 193.3 57) (width 0.5) (layer "F.Cu") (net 3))
 (segment (start 194.15 13.15) (end 194.15 20.7) (width 0.5) (layer "F.Cu") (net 3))
 (segment (start 193.55 12.55) (end 194.15 13.15) (width 0.5) (layer "F.Cu") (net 3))
 (segment (start 103.85 74.8) (end 102.9 75.75) (width 0.5) (layer "F.Cu") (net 3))
 (segment (start 193.4 102.95) (end 193.4 109.35) (width 0.5) (layer "F.Cu") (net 3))
 (segment (start 99.9 70.8) (end 99.9 14.05) (width 0.5) (layer "F.Cu") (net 3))
 (segment (start 103.55 48.1) (end 193.25 48.1) (width 0.5) (layer "F.Cu") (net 3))
 (via (at 83.6 52.95) (size 0.8) (drill 0.4) (layers "F.Cu" "B.Cu") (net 3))
 (via (at 87.35 70.55) (size 0.8) (drill 0.4) (layers "F.Cu" "B.Cu") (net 3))
 (segment (start 87.35 56.55) (end 87.35 70.55) (width 0.5) (layer "B.Cu") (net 3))
 (segment (start 83.6 52.95) (end 83.75 52.95) (width 0.5) (layer "B.Cu") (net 3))
 (segment (start 83.75 52.95) (end 87.35 56.55) (width 0.5) (layer "B.Cu") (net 3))
 (segment (start 85.719 19.72) (end 81.38 19.72) (width 0.15) (layer "F.Cu") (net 8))
 (segment (start 77.75 45.55) (end 77.7 45.6) (width 0.15) (layer "F.Cu") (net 8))
 (segment (start 79.5 45.55) (end 77.75 45.55) (width 0.15) (layer "F.Cu") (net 8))
 (segment (start 76.45 47.6) (end 76.8 47.95) (width 0.15) (layer "F.Cu") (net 8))
 (segment (start 81.38 19.72) (end 81.05 20.05) (width 0.15) (layer "F.Cu") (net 8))
 (segment (start 76.8 47.95) (end 77.9 47.95) (width 0.15) (layer "F.Cu") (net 8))
 (via (at 77.7 45.6) (size 0.8) (drill 0.4) (layers "F.Cu" "B.Cu") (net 8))
 (via (at 81.05 20.05) (size 0.8) (drill 0.4) (layers "F.Cu" "B.Cu") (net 8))
 (via (at 79.5 45.55) (size 0.8) (drill 0.4) (layers "F.Cu" "B.Cu") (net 8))
 (via (at 76.45 47.6) (size 0.8) (drill 0.4) (layers "F.Cu" "B.Cu") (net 8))
 (segment (start 76.45 46.85) (end 76.45 47.6) (width 0.15) (layer "B.Cu") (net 8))
 (segment (start 79.5 21.6) (end 79.5 45.4) (width 0.15) (layer "B.Cu") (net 8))
 (segment (start 79.5 45.4) (end 79.5 45.55) (width 0.15) (layer "B.Cu") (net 8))
 (segment (start 77.7 45.6) (end 76.45 46.85) (width 0.15) (layer "B.Cu") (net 8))
 (segment (start 81.05 20.05) (end 79.5 21.6) (width 0.15) (layer "B.Cu") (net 8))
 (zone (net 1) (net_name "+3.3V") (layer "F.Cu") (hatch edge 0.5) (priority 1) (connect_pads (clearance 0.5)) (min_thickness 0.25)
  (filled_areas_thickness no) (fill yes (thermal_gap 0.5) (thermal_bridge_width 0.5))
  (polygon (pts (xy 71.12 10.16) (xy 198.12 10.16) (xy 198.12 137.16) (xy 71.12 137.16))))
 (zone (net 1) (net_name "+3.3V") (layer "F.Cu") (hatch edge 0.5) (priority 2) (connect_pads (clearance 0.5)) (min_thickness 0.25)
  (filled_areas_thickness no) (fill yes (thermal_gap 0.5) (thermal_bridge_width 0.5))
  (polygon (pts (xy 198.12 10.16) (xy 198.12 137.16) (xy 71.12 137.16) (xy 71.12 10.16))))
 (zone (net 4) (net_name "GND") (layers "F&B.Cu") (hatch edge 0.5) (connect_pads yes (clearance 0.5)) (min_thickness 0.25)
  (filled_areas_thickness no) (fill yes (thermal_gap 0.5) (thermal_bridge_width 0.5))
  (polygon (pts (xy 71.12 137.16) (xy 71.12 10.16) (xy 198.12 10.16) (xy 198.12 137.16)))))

